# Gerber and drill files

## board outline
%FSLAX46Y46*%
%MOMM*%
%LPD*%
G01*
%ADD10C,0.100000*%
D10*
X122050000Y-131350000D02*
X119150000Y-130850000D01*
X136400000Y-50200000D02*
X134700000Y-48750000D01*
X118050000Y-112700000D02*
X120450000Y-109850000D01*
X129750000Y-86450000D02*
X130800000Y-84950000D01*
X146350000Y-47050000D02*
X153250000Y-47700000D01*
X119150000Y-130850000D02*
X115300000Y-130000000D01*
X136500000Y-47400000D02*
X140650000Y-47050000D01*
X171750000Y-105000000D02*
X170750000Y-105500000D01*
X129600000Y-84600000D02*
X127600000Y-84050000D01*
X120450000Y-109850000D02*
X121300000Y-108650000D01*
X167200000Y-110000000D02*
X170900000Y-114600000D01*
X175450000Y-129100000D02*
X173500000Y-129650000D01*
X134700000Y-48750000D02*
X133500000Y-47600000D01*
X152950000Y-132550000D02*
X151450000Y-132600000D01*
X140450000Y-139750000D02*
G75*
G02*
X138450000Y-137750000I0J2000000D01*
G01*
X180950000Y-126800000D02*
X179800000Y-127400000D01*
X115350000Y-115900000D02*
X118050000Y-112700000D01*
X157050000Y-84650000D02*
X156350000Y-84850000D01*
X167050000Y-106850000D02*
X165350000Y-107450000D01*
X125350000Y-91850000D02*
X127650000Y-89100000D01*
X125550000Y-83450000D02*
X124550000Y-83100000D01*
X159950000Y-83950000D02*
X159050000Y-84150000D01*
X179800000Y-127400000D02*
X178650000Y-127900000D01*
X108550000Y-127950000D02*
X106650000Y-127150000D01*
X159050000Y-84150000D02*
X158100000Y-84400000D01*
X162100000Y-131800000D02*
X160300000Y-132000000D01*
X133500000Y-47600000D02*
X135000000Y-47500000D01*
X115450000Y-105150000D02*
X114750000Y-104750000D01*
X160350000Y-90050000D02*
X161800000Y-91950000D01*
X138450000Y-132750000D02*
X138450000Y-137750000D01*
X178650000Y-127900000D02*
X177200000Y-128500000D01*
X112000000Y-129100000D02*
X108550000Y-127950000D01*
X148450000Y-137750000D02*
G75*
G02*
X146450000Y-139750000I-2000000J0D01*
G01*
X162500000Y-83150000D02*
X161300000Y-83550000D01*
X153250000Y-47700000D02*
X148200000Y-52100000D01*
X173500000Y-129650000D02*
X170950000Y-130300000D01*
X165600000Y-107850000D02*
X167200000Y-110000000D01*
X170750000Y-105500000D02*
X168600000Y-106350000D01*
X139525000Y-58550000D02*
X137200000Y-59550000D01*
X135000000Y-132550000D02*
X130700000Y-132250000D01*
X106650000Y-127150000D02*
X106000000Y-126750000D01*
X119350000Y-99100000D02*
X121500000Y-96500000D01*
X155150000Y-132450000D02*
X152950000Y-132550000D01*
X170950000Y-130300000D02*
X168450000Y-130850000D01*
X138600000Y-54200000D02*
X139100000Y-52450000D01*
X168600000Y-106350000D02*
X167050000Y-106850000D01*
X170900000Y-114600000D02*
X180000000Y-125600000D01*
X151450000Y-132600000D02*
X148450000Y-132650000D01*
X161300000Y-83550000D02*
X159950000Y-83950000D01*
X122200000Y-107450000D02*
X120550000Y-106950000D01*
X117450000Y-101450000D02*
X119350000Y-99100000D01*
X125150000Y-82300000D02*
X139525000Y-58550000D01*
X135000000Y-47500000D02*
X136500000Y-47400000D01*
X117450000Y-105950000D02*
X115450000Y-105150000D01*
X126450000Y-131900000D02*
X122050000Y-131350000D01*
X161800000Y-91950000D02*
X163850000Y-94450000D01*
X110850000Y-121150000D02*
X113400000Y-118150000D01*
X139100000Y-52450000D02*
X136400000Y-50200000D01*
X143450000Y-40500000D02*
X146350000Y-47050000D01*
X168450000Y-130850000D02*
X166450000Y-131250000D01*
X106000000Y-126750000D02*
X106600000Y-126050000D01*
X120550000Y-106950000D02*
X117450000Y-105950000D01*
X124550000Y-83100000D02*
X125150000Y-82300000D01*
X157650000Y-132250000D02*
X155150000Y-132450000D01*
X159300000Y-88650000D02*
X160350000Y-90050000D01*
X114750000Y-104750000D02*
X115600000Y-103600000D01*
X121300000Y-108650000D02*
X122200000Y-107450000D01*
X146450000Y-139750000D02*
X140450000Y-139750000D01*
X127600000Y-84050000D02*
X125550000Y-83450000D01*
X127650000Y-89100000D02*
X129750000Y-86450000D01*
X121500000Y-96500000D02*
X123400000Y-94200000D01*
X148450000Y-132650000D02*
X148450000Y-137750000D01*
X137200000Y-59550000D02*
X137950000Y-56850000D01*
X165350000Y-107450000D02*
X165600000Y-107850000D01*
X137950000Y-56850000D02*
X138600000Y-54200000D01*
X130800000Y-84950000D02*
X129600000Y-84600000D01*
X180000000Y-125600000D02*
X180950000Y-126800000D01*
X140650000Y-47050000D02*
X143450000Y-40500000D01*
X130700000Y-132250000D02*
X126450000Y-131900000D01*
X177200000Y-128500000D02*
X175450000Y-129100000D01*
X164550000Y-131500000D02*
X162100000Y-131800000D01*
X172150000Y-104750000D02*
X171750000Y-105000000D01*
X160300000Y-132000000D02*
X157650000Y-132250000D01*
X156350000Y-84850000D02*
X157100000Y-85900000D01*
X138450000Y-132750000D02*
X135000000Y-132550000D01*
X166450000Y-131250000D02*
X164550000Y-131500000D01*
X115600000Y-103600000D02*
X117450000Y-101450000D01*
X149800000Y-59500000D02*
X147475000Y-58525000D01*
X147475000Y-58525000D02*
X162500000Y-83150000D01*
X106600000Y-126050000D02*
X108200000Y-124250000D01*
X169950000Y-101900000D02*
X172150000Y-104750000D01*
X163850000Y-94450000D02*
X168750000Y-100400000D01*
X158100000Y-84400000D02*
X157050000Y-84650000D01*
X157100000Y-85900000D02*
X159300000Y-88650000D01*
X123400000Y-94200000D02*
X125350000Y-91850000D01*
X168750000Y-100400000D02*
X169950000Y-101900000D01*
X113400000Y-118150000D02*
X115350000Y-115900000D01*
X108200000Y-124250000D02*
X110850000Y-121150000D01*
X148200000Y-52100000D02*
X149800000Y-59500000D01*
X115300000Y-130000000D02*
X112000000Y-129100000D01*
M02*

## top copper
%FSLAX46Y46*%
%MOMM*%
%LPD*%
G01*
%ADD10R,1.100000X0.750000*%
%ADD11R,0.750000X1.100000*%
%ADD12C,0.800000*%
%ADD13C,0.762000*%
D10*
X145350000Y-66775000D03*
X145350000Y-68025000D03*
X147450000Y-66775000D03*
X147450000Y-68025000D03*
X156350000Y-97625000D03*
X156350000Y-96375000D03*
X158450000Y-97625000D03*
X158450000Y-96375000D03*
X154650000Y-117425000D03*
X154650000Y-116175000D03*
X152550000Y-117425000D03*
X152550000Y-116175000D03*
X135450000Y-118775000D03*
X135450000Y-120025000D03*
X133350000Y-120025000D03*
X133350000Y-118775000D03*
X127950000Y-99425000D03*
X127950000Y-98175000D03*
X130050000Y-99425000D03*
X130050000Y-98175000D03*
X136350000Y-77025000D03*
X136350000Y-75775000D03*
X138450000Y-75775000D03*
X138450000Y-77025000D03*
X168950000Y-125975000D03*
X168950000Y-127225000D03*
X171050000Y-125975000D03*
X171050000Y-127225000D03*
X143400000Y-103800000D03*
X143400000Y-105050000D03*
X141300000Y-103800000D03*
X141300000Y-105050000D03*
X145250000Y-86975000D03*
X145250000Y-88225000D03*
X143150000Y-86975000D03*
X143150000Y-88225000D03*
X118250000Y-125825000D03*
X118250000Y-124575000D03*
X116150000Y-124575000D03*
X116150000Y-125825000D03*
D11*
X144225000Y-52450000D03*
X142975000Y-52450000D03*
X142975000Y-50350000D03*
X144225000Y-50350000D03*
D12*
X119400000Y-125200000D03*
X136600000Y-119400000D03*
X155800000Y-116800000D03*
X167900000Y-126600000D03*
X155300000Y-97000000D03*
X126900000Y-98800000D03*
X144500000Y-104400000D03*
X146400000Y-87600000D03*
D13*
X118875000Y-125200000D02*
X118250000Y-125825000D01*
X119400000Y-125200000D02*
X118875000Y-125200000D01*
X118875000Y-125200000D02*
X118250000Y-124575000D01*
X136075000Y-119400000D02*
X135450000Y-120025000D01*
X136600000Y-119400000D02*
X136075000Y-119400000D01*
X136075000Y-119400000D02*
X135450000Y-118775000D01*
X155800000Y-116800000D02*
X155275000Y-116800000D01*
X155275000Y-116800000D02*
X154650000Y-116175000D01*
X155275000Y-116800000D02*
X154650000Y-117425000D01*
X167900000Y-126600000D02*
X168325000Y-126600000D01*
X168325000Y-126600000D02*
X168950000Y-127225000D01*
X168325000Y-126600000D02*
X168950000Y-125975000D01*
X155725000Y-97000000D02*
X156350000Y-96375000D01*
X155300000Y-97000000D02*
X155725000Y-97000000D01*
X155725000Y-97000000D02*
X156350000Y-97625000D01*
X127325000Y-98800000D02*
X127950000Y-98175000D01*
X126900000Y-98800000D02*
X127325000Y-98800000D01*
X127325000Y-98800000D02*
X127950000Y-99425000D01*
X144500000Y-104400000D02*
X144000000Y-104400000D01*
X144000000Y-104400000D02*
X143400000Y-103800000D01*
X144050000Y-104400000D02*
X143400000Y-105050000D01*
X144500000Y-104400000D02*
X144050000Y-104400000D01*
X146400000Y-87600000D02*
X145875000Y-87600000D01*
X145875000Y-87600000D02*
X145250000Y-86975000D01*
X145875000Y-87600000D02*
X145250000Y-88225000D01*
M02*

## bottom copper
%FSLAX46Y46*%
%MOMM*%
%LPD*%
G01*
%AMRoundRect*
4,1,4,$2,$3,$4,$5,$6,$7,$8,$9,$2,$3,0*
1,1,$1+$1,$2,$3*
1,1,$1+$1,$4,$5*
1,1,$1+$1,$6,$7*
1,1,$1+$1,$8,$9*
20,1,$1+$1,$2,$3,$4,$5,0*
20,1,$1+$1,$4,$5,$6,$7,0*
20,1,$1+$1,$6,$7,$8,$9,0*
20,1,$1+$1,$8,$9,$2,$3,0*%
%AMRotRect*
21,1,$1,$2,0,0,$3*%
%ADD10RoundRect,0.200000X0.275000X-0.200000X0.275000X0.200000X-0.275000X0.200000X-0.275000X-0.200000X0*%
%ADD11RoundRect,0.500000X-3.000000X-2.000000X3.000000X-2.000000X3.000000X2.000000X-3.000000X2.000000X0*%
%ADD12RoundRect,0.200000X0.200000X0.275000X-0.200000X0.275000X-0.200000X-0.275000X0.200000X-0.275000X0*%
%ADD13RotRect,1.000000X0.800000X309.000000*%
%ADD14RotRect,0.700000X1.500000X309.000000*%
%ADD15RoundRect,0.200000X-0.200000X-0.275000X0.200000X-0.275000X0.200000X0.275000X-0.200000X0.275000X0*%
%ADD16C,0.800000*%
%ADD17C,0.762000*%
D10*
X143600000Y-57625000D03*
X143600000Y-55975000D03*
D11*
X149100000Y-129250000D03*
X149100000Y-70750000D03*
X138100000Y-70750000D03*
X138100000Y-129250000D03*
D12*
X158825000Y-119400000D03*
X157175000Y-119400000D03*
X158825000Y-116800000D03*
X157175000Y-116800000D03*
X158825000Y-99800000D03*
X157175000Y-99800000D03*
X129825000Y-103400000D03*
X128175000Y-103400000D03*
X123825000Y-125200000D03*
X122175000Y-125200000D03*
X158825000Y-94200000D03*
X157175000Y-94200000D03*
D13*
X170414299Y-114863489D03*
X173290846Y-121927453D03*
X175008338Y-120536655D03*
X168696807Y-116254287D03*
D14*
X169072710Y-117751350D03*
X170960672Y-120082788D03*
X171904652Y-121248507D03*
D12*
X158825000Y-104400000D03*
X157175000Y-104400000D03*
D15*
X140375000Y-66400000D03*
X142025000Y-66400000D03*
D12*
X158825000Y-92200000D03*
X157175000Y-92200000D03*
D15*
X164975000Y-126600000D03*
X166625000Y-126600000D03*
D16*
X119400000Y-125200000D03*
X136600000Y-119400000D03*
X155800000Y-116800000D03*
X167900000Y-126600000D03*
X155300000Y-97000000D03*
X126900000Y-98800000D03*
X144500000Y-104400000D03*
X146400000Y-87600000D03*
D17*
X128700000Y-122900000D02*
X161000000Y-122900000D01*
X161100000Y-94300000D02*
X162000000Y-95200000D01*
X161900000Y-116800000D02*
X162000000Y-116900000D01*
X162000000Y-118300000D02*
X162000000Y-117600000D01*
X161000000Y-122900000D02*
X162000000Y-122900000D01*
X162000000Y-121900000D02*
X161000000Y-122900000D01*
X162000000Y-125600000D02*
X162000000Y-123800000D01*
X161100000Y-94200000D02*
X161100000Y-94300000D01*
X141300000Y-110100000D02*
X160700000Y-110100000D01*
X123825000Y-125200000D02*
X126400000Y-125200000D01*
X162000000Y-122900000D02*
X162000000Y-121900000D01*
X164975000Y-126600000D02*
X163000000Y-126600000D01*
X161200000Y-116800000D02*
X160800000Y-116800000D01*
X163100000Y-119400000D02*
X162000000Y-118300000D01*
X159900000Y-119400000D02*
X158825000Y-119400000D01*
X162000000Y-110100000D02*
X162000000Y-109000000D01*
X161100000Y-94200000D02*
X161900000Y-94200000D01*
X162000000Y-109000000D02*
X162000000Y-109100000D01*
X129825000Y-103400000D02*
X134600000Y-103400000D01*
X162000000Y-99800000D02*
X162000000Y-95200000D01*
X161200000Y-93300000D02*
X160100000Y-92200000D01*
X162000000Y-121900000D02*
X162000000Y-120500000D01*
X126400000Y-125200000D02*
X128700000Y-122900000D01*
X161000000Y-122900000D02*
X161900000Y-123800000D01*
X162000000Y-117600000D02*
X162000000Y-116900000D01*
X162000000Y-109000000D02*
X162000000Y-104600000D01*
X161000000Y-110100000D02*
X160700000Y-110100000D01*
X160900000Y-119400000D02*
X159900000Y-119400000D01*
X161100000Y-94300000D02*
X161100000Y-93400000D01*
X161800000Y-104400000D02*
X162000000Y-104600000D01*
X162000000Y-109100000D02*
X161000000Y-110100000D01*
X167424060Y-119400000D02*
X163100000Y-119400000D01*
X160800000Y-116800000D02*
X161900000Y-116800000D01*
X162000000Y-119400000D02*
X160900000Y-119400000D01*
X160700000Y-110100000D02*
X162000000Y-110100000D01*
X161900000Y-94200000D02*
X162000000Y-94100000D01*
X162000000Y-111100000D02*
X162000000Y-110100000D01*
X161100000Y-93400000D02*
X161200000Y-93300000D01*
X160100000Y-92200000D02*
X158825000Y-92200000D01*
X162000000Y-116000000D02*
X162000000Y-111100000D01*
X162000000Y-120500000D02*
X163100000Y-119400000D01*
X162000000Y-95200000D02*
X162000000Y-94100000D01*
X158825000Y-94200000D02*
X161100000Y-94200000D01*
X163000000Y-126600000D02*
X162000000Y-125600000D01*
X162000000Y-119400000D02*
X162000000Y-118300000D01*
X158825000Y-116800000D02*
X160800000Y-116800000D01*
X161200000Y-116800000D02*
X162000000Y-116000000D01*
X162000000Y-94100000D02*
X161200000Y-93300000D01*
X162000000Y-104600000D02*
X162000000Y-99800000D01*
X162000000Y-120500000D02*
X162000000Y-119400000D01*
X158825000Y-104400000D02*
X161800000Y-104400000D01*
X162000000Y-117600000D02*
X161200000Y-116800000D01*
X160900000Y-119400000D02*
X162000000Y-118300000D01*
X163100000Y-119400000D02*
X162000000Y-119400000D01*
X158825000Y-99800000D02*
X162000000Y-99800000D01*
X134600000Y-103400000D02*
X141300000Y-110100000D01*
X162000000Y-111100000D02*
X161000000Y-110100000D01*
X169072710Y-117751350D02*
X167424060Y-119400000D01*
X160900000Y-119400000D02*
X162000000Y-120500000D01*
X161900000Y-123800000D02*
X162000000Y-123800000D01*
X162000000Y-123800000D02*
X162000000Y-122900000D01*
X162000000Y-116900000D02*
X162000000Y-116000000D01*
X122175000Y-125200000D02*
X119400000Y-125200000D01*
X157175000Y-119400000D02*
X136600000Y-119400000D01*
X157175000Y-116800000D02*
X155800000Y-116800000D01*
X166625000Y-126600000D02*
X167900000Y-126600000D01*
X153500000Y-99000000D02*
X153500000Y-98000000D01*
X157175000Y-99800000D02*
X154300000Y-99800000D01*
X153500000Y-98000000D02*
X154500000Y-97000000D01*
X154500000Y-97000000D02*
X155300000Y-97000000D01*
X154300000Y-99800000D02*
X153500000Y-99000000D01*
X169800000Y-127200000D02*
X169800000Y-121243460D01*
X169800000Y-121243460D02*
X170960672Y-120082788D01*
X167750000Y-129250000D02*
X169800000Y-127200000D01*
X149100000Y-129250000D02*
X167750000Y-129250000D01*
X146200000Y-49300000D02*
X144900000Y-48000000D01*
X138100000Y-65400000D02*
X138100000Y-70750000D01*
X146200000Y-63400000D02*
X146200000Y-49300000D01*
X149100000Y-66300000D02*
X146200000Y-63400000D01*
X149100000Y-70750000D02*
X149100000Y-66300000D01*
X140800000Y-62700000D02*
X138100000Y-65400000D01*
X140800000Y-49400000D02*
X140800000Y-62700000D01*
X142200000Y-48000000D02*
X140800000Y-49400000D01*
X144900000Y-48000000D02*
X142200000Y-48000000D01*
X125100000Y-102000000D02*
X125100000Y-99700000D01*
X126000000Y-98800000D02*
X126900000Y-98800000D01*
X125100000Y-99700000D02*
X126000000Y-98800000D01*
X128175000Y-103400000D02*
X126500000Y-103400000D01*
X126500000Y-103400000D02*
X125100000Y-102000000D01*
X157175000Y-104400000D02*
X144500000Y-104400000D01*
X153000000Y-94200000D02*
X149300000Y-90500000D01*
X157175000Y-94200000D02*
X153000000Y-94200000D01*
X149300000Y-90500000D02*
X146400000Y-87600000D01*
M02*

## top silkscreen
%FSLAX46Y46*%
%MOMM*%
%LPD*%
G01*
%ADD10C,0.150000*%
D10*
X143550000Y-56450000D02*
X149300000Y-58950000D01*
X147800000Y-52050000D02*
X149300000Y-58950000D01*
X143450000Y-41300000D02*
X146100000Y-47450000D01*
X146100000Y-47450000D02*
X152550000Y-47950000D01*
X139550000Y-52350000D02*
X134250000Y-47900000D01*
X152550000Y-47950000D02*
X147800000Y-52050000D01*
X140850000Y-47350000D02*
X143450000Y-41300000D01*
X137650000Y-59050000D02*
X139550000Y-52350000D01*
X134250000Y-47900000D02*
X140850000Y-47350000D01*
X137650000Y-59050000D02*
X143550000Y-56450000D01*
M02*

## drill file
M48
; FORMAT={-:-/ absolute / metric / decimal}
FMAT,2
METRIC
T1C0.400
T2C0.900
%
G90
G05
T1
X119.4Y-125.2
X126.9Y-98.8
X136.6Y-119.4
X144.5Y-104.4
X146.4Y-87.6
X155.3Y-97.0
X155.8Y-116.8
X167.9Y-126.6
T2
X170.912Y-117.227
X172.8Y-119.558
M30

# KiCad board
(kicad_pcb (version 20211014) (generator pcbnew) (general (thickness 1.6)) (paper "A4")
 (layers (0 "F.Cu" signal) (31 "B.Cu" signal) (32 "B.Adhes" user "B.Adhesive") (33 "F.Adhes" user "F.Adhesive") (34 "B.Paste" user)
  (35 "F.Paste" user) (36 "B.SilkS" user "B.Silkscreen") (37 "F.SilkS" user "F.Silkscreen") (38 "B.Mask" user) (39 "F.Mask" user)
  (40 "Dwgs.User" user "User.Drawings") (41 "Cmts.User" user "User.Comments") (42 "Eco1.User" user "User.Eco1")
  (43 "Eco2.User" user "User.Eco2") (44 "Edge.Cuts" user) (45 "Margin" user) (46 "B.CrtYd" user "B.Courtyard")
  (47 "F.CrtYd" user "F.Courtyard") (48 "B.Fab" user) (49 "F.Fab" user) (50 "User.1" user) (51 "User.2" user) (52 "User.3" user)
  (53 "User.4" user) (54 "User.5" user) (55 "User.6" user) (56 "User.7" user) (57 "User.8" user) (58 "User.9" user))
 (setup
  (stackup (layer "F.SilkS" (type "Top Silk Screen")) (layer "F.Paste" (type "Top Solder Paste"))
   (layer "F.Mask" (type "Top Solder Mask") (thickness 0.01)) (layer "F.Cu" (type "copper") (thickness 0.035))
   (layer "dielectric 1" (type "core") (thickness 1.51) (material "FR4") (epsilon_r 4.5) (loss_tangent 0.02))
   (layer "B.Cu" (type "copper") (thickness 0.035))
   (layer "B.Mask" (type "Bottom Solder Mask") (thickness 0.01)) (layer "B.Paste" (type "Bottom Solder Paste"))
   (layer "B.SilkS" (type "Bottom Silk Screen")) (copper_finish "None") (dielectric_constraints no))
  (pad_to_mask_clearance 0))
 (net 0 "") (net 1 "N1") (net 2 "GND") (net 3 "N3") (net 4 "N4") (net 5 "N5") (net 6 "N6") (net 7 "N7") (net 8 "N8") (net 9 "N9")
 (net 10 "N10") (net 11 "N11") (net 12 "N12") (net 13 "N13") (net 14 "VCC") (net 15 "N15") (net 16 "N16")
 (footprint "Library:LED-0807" (layer "F.Cu") (at 146.4 67.4)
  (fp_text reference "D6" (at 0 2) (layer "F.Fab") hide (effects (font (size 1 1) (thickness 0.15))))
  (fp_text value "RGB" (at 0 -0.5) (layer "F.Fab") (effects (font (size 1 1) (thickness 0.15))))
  (pad "1" smd rect locked (at -1.05 -0.625) (size 1.1 0.75) (layers "F.Cu" "F.Paste" "F.Mask") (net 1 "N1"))
  (pad "1" smd rect locked (at -1.05 0.625) (size 1.1 0.75) (layers "F.Cu" "F.Paste" "F.Mask") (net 1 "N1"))
  (pad "2" smd rect locked (at 1.05 -0.625) (size 1.1 0.75) (layers "F.Cu" "F.Paste" "F.Mask") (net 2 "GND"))
  (pad "2" smd rect locked (at 1.05 0.625) (size 1.1 0.75) (layers "F.Cu" "F.Paste" "F.Mask") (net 2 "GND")))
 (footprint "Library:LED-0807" (layer "F.Cu") (at 157.4 97)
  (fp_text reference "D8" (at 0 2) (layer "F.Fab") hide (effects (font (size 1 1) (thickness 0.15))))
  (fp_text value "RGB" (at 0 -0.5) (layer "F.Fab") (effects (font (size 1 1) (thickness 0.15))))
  (pad "1" smd rect locked (at -1.05 0.625) (size 1.1 0.75) (layers "F.Cu" "F.Paste" "F.Mask") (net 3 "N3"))
  (pad "1" smd rect locked (at -1.05 -0.625) (size 1.1 0.75) (layers "F.Cu" "F.Paste" "F.Mask") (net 3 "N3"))
  (pad "2" smd rect locked (at 1.05 0.625) (size 1.1 0.75) (layers "F.Cu" "F.Paste" "F.Mask") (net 2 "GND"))
  (pad "2" smd rect locked (at 1.05 -0.625) (size 1.1 0.75) (layers "F.Cu" "F.Paste" "F.Mask") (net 2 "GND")))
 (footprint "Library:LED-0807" (layer "F.Cu") (at 153.6 116.8 180)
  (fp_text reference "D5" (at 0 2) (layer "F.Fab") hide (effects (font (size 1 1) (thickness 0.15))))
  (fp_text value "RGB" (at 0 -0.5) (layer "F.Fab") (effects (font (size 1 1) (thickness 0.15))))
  (pad "1" smd rect locked (at -1.05 -0.625 180) (size 1.1 0.75) (layers "F.Cu" "F.Paste" "F.Mask") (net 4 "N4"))
  (pad "1" smd rect locked (at -1.05 0.625 180) (size 1.1 0.75) (layers "F.Cu" "F.Paste" "F.Mask") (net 4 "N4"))
  (pad "2" smd rect locked (at 1.05 -0.625 180) (size 1.1 0.75) (layers "F.Cu" "F.Paste" "F.Mask") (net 2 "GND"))
  (pad "2" smd rect locked (at 1.05 0.625 180) (size 1.1 0.75) (layers "F.Cu" "F.Paste" "F.Mask") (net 2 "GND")))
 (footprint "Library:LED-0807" (layer "F.Cu") (at 134.4 119.4 180)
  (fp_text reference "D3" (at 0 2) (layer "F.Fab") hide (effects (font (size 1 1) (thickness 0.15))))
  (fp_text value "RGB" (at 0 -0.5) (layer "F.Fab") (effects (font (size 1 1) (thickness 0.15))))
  (pad "1" smd rect locked (at -1.05 0.625 180) (size 1.1 0.75) (layers "F.Cu" "F.Paste" "F.Mask") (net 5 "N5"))
  (pad "1" smd rect locked (at -1.05 -0.625 180) (size 1.1 0.75) (layers "F.Cu" "F.Paste" "F.Mask") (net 5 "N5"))
  (pad "2" smd rect locked (at 1.05 -0.625 180) (size 1.1 0.75) (layers "F.Cu" "F.Paste" "F.Mask") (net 2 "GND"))
  (pad "2" smd rect locked (at 1.05 0.625 180) (size 1.1 0.75) (layers "F.Cu" "F.Paste" "F.Mask") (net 2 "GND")))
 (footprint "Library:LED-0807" (layer "F.Cu") (at 129 98.8)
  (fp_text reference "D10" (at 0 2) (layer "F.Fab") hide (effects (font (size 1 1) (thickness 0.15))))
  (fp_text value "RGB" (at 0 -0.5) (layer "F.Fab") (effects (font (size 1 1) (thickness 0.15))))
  (pad "1" smd rect locked (at -1.05 0.625) (size 1.1 0.75) (layers "F.Cu" "F.Paste" "F.Mask") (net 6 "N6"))
  (pad "1" smd rect locked (at -1.05 -0.625) (size 1.1 0.75) (layers "F.Cu" "F.Paste" "F.Mask") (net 6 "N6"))
  (pad "2" smd rect locked (at 1.05 0.625) (size 1.1 0.75) (layers "F.Cu" "F.Paste" "F.Mask") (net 2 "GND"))
  (pad "2" smd rect locked (at 1.05 -0.625) (size 1.1 0.75) (layers "F.Cu" "F.Paste" "F.Mask") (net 2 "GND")))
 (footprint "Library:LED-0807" (layer "F.Cu") (at 137.4 76.4)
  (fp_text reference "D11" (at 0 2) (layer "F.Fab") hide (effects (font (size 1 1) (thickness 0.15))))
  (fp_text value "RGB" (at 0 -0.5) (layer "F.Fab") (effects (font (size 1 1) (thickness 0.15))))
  (pad "1" smd rect locked (at -1.05 0.625) (size 1.1 0.75) (layers "F.Cu" "F.Paste" "F.Mask") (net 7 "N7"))
  (pad "1" smd rect locked (at -1.05 -0.625) (size 1.1 0.75) (layers "F.Cu" "F.Paste" "F.Mask") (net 7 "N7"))
  (pad "2" smd rect locked (at 1.05 -0.625) (size 1.1 0.75) (layers "F.Cu" "F.Paste" "F.Mask") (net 2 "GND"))
  (pad "2" smd rect locked (at 1.05 0.625) (size 1.1 0.75) (layers "F.Cu" "F.Paste" "F.Mask") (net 2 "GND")))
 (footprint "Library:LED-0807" (layer "F.Cu") (at 170 126.6)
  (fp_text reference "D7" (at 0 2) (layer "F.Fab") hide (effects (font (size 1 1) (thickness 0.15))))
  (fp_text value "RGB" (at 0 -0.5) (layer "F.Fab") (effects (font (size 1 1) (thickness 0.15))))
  (pad "1" smd rect locked (at -1.05 -0.625) (size 1.1 0.75) (layers "F.Cu" "F.Paste" "F.Mask") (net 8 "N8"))
  (pad "1" smd rect locked (at -1.05 0.625) (size 1.1 0.75) (layers "F.Cu" "F.Paste" "F.Mask") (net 8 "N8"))
  (pad "2" smd rect locked (at 1.05 -0.625) (size 1.1 0.75) (layers "F.Cu" "F.Paste" "F.Mask") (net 2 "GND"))
  (pad "2" smd rect locked (at 1.05 0.625) (size 1.1 0.75) (layers "F.Cu" "F.Paste" "F.Mask") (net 2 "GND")))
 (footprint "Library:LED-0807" (layer "F.Cu") (at 142.35 104.425 180)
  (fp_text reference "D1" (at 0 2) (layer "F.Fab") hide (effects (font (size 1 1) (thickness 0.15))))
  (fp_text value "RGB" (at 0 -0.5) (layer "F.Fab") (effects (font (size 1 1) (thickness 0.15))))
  (pad "1" smd rect locked (at -1.05 0.625 180) (size 1.1 0.75) (layers "F.Cu" "F.Paste" "F.Mask") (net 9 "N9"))
  (pad "1" smd rect locked (at -1.05 -0.625 180) (size 1.1 0.75) (layers "F.Cu" "F.Paste" "F.Mask") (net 9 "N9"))
  (pad "2" smd rect locked (at 1.05 0.625 180) (size 1.1 0.75) (layers "F.Cu" "F.Paste" "F.Mask") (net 2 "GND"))
  (pad "2" smd rect locked (at 1.05 -0.625 180) (size 1.1 0.75) (layers "F.Cu" "F.Paste" "F.Mask") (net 2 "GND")))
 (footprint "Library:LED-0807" (layer "F.Cu") (at 144.2 87.6 180)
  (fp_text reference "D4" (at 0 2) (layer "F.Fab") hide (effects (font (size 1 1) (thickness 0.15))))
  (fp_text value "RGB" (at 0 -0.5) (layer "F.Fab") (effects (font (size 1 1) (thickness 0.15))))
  (pad "1" smd rect locked (at -1.05 0.625 180) (size 1.1 0.75) (layers "F.Cu" "F.Paste" "F.Mask") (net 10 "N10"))
  (pad "1" smd rect locked (at -1.05 -0.625 180) (size 1.1 0.75) (layers "F.Cu" "F.Paste" "F.Mask") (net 10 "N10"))
  (pad "2" smd rect locked (at 1.05 0.625 180) (size 1.1 0.75) (layers "F.Cu" "F.Paste" "F.Mask") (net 2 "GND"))
  (pad "2" smd rect locked (at 1.05 -0.625 180) (size 1.1 0.75) (layers "F.Cu" "F.Paste" "F.Mask") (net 2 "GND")))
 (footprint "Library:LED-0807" (layer "F.Cu") (at 117.2 125.2 180)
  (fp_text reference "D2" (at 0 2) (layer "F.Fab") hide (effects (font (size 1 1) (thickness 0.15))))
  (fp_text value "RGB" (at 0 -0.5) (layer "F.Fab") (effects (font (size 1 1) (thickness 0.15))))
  (pad "1" smd rect locked (at -1.05 -0.625 180) (size 1.1 0.75) (layers "F.Cu" "F.Paste" "F.Mask") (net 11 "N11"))
  (pad "1" smd rect locked (at -1.05 0.625 180) (size 1.1 0.75) (layers "F.Cu" "F.Paste" "F.Mask") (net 11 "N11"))
  (pad "2" smd rect locked (at 1.05 0.625 180) (size 1.1 0.75) (layers "F.Cu" "F.Paste" "F.Mask") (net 2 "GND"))
  (pad "2" smd rect locked (at 1.05 -0.625 180) (size 1.1 0.75) (layers "F.Cu" "F.Paste" "F.Mask") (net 2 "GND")))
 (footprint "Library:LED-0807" (layer "F.Cu") (at 143.6 51.4 90)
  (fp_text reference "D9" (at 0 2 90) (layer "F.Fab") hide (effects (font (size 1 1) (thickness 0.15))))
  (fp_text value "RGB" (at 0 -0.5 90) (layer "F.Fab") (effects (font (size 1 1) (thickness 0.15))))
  (pad "1" smd rect locked (at -1.05 0.625 90) (size 1.1 0.75) (layers "F.Cu" "F.Paste" "F.Mask") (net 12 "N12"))
  (pad "1" smd rect locked (at -1.05 -0.625 90) (size 1.1 0.75) (layers "F.Cu" "F.Paste" "F.Mask") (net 12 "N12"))
  (pad "2" smd rect locked (at 1.05 -0.625 90) (size 1.1 0.75) (layers "F.Cu" "F.Paste" "F.Mask") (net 2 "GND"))
  (pad "2" smd rect locked (at 1.05 0.625 90) (size 1.1 0.75) (layers "F.Cu" "F.Paste" "F.Mask") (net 2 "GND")))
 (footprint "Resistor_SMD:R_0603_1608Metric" (layer "B.Cu") (at 143.6 56.8 90)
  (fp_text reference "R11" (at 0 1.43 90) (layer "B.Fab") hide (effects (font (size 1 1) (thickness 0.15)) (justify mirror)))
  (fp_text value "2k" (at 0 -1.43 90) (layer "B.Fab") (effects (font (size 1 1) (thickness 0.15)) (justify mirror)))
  (pad "1" smd roundrect locked (at -0.825 0 90) (size 0.8 0.95) (layers "B.Cu" "B.Paste" "B.Mask") (roundrect_rratio 0.25) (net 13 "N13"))
  (pad "2" smd roundrect locked (at 0.825 0 90) (size 0.8 0.95) (layers "B.Cu" "B.Paste" "B.Mask") (roundrect_rratio 0.25) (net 12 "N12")))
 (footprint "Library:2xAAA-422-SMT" (layer "B.Cu") (at 143.6 100)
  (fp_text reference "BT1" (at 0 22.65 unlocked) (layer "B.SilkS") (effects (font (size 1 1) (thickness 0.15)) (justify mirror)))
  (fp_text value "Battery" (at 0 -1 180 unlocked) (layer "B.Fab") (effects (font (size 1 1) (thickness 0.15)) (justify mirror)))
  (pad "1" smd roundrect (at 5.5 29.25) (size 7 5) (layers "B.Cu" "B.Paste" "B.Mask") (roundrect_rratio 0.1) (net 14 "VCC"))
  (pad "2" smd roundrect (at 5.5 -29.25) (size 7 5) (layers "B.Cu" "B.Paste" "B.Mask") (roundrect_rratio 0.1) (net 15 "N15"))
  (pad "2" smd roundrect (at -5.5 -29.25) (size 7 5) (layers "B.Cu" "B.Paste" "B.Mask") (roundrect_rratio 0.1) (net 15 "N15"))
  (pad "3" smd roundrect (at -5.5 29.25) (size 7 5) (layers "B.Cu" "B.Paste" "B.Mask") (roundrect_rratio 0.1) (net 2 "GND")))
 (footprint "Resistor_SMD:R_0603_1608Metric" (layer "B.Cu") (at 158 119.4 180)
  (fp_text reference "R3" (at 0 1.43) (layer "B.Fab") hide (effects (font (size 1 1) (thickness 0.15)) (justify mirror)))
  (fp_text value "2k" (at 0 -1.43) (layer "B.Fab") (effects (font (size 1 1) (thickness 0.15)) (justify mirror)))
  (pad "1" smd roundrect locked (at -0.825 0 180) (size 0.8 0.95) (layers "B.Cu" "B.Paste" "B.Mask") (roundrect_rratio 0.25) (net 13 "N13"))
  (pad "2" smd roundrect locked (at 0.825 0 180) (size 0.8 0.95) (layers "B.Cu" "B.Paste" "B.Mask") (roundrect_rratio 0.25) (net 5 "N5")))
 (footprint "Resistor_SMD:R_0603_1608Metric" (layer "B.Cu") (at 158 116.8 180)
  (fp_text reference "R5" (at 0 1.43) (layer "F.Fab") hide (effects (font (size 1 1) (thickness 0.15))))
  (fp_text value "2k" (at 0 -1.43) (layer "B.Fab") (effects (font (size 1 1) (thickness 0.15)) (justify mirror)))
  (pad "1" smd roundrect locked (at -0.825 0 180) (size 0.8 0.95) (layers "B.Cu" "B.Paste" "B.Mask") (roundrect_rratio 0.25) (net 13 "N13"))
  (pad "2" smd roundrect locked (at 0.825 0 180) (size 0.8 0.95) (layers "B.Cu" "B.Paste" "B.Mask") (roundrect_rratio 0.25) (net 4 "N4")))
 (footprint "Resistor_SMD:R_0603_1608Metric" (layer "B.Cu") (at 158 99.8 180)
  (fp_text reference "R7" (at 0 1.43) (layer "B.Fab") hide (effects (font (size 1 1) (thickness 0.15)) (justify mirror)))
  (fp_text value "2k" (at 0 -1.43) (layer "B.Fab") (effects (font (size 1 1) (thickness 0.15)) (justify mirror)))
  (pad "1" smd roundrect locked (at -0.825 0 180) (size 0.8 0.95) (layers "B.Cu" "B.Paste" "B.Mask") (roundrect_rratio 0.25) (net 13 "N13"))
  (pad "2" smd roundrect locked (at 0.825 0 180) (size 0.8 0.95) (layers "B.Cu" "B.Paste" "B.Mask") (roundrect_rratio 0.25) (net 3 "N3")))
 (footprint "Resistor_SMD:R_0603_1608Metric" (layer "B.Cu") (at 129 103.4 180)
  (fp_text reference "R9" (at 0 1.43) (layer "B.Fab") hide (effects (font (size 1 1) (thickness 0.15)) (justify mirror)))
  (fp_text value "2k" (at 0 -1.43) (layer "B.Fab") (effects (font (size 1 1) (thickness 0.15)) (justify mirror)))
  (pad "1" smd roundrect locked (at -0.825 0 180) (size 0.8 0.95) (layers "B.Cu" "B.Paste" "B.Mask") (roundrect_rratio 0.25) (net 13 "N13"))
  (pad "2" smd roundrect locked (at 0.825 0 180) (size 0.8 0.95) (layers "B.Cu" "B.Paste" "B.Mask") (roundrect_rratio 0.25) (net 6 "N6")))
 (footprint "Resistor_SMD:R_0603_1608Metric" (layer "B.Cu") (at 123 125.2 180)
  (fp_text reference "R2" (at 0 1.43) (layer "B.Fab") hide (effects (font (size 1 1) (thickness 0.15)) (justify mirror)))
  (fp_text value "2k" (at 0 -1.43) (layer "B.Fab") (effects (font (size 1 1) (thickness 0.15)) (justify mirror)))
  (pad "1" smd roundrect locked (at -0.825 0 180) (size 0.8 0.95) (layers "B.Cu" "B.Paste" "B.Mask") (roundrect_rratio 0.25) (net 13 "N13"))
  (pad "2" smd roundrect locked (at 0.825 0 180) (size 0.8 0.95) (layers "B.Cu" "B.Paste" "B.Mask") (roundrect_rratio 0.25) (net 11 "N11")))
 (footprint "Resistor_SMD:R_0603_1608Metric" (layer "B.Cu") (at 158 94.2 180)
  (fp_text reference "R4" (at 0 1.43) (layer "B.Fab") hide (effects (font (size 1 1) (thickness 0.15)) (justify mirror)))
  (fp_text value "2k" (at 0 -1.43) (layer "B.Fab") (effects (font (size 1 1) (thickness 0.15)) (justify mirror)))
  (pad "1" smd roundrect locked (at -0.825 0 180) (size 0.8 0.95) (layers "B.Cu" "B.Paste" "B.Mask") (roundrect_rratio 0.25) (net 13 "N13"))
  (pad "2" smd roundrect locked (at 0.825 0 180) (size 0.8 0.95) (layers "B.Cu" "B.Paste" "B.Mask") (roundrect_rratio 0.25) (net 10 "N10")))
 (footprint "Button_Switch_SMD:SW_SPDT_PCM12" (layer "B.Cu") (at 171.6 118.6 -51)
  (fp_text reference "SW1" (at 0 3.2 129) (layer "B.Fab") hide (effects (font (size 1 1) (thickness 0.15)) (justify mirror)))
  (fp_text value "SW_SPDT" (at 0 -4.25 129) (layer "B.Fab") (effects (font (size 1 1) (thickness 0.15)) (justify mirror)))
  (pad "" smd rect locked (at -3.65 -1.43 309) (size 1 0.8) (layers "B.Cu" "B.Paste" "B.Mask"))
  (pad "" np_thru_hole circle locked (at 1.5 -0.33 309) (size 0.9 0.9) (drill 0.9) (layers *.Cu *.Mask))
  (pad "" smd rect locked (at 3.65 0.78 309) (size 1 0.8) (layers "B.Cu" "B.Paste" "B.Mask"))
  (pad "" np_thru_hole circle locked (at -1.5 -0.33 309) (size 0.9 0.9) (drill 0.9) (layers *.Cu *.Mask))
  (pad "" smd rect locked (at 3.65 -1.43 309) (size 1 0.8) (layers "B.Cu" "B.Paste" "B.Mask"))
  (pad "" smd rect locked (at -3.65 0.78 309) (size 1 0.8) (layers "B.Cu" "B.Paste" "B.Mask"))
  (pad "1" smd rect locked (at -2.25 1.43 309) (size 0.7 1.5) (layers "B.Cu" "B.Paste" "B.Mask") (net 13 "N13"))
  (pad "2" smd rect locked (at 0.75 1.43 309) (size 0.7 1.5) (layers "B.Cu" "B.Paste" "B.Mask") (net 14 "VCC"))
  (pad "3" smd rect locked (at 2.25 1.43 309) (size 0.7 1.5) (layers "B.Cu" "B.Paste" "B.Mask") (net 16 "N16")))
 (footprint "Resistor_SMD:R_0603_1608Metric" (layer "B.Cu") (at 158 104.4 180)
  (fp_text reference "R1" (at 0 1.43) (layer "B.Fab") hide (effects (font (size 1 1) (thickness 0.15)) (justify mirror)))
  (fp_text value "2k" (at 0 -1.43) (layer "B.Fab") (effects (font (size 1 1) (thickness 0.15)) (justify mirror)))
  (pad "1" smd roundrect locked (at -0.825 0 180) (size 0.8 0.95) (layers "B.Cu" "B.Paste" "B.Mask") (roundrect_rratio 0.25) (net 13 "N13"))
  (pad "2" smd roundrect locked (at 0.825 0 180) (size 0.8 0.95) (layers "B.Cu" "B.Paste" "B.Mask") (roundrect_rratio 0.25) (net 9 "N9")))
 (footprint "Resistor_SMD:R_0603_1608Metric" (layer "B.Cu") (at 141.2 66.4)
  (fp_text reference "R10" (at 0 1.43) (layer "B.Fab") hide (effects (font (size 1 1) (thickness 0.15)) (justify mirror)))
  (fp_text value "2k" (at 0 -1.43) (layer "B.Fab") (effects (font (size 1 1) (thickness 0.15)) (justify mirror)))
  (pad "1" smd roundrect locked (at -0.825 0) (size 0.8 0.95) (layers "B.Cu" "B.Paste" "B.Mask") (roundrect_rratio 0.25) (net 13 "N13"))
  (pad "2" smd roundrect locked (at 0.825 0) (size 0.8 0.95) (layers "B.Cu" "B.Paste" "B.Mask") (roundrect_rratio 0.25) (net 1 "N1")))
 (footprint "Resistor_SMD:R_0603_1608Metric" (layer "B.Cu") (at 158 92.2 180)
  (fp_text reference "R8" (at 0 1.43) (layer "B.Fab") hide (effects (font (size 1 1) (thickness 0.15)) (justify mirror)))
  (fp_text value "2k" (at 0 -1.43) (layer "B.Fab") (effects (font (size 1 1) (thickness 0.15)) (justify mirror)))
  (pad "1" smd roundrect locked (at -0.825 0 180) (size 0.8 0.95) (layers "B.Cu" "B.Paste" "B.Mask") (roundrect_rratio 0.25) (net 13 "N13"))
  (pad "2" smd roundrect locked (at 0.825 0 180) (size 0.8 0.95) (layers "B.Cu" "B.Paste" "B.Mask") (roundrect_rratio 0.25) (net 7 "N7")))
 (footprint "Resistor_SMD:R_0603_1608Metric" (layer "B.Cu") (at 165.8 126.6)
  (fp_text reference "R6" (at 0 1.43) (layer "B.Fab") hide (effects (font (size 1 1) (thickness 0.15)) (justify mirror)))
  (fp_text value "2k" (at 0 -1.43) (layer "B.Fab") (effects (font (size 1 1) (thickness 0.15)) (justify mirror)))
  (pad "1" smd roundrect locked (at -0.825 0) (size 0.8 0.95) (layers "B.Cu" "B.Paste" "B.Mask") (roundrect_rratio 0.25) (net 13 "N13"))
  (pad "2" smd roundrect locked (at 0.825 0) (size 0.8 0.95) (layers "B.Cu" "B.Paste" "B.Mask") (roundrect_rratio 0.25) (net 8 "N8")))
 (gr_line (start 143.55 56.45) (end 149.3 58.95) (layer "F.SilkS") (width 0.15))
 (gr_line (start 147.8 52.05) (end 149.3 58.95) (layer "F.SilkS") (width 0.15))
 (gr_line (start 143.45 41.3) (end 146.1 47.45) (layer "F.SilkS") (width 0.15))
 (gr_line (start 146.1 47.45) (end 152.55 47.95) (layer "F.SilkS") (width 0.15))
 (gr_line (start 139.55 52.35) (end 134.25 47.9) (layer "F.SilkS") (width 0.15))
 (gr_line (start 152.55 47.95) (end 147.8 52.05) (layer "F.SilkS") (width 0.15))
 (gr_line (start 140.85 47.35) (end 143.45 41.3) (layer "F.SilkS") (width 0.15))
 (gr_line (start 137.65 59.05) (end 139.55 52.35) (layer "F.SilkS") (width 0.15))
 (gr_line (start 134.25 47.9) (end 140.85 47.35) (layer "F.SilkS") (width 0.15))
 (gr_line (start 137.65 59.05) (end 143.55 56.45) (layer "F.SilkS") (width 0.15))
 (gr_line (start 122.05 131.35) (end 119.15 130.85) (layer "Edge.Cuts") (width 0.1))
 (gr_line (start 136.4 50.2) (end 134.7 48.75) (layer "Edge.Cuts") (width 0.1))
 (gr_line (start 118.05 112.7) (end 120.45 109.85) (layer "Edge.Cuts") (width 0.1))
 (gr_line (start 129.75 86.45) (end 130.8 84.95) (layer "Edge.Cuts") (width 0.1))
 (gr_line (start 146.35 47.05) (end 153.25 47.7) (layer "Edge.Cuts") (width 0.1))
 (gr_line (start 119.15 130.85) (end 115.3 130) (layer "Edge.Cuts") (width 0.1))
 (gr_line (start 136.5 47.4) (end 140.65 47.05) (layer "Edge.Cuts") (width 0.1))
 (gr_line (start 171.75 105) (end 170.75 105.5) (layer "Edge.Cuts") (width 0.1))
 (gr_line (start 129.6 84.6) (end 127.6 84.05) (layer "Edge.Cuts") (width 0.1))
 (gr_line (start 120.45 109.85) (end 121.3 108.65) (layer "Edge.Cuts") (width 0.1))
 (gr_line (start 167.2 110) (end 170.9 114.6) (layer "Edge.Cuts") (width 0.1))
 (gr_line (start 175.45 129.1) (end 173.5 129.65) (layer "Edge.Cuts") (width 0.1))
 (gr_line (start 134.7 48.75) (end 133.5 47.6) (layer "Edge.Cuts") (width 0.1))
 (gr_line (start 152.95 132.55) (end 151.45 132.6) (layer "Edge.Cuts") (width 0.1))
 (gr_arc (start 140.45 139.75) (mid 139.035786 139.164214) (end 138.45 137.75) (layer "Edge.Cuts") (width 0.1))
 (gr_line (start 180.95 126.8) (end 179.8 127.4) (layer "Edge.Cuts") (width 0.1))
 (gr_line (start 115.35 115.9) (end 118.05 112.7) (layer "Edge.Cuts") (width 0.1))
 (gr_line (start 157.05 84.65) (end 156.35 84.85) (layer "Edge.Cuts") (width 0.1))
 (gr_line (start 167.05 106.85) (end 165.35 107.45) (layer "Edge.Cuts") (width 0.1))
 (gr_line (start 125.35 91.85) (end 127.65 89.1) (layer "Edge.Cuts") (width 0.1))
 (gr_line (start 125.55 83.45) (end 124.55 83.1) (layer "Edge.Cuts") (width 0.1))
 (gr_line (start 159.95 83.95) (end 159.05 84.15) (layer "Edge.Cuts") (width 0.1))
 (gr_line (start 179.8 127.4) (end 178.65 127.9) (layer "Edge.Cuts") (width 0.1))
 (gr_line (start 108.55 127.95) (end 106.65 127.15) (layer "Edge.Cuts") (width 0.1))
 (gr_line (start 159.05 84.15) (end 158.1 84.4) (layer "Edge.Cuts") (width 0.1))
 (gr_line (start 162.1 131.8) (end 160.3 132) (layer "Edge.Cuts") (width 0.1))
 (gr_line (start 133.5 47.6) (end 135 47.5) (layer "Edge.Cuts") (width 0.1))
 (gr_line (start 115.45 105.15) (end 114.75 104.75) (layer "Edge.Cuts") (width 0.1))
 (gr_line (start 160.35 90.05) (end 161.8 91.95) (layer "Edge.Cuts") (width 0.1))
 (gr_line (start 138.45 132.75) (end 138.45 137.75) (layer "Edge.Cuts") (width 0.1))
 (gr_line (start 178.65 127.9) (end 177.2 128.5) (layer "Edge.Cuts") (width 0.1))
 (gr_line (start 112 129.1) (end 108.55 127.95) (layer "Edge.Cuts") (width 0.1))
 (gr_arc (start 148.45 137.75) (mid 147.864214 139.164214) (end 146.45 139.75) (layer "Edge.Cuts") (width 0.1))
 (gr_line (start 162.5 83.15) (end 161.3 83.55) (layer "Edge.Cuts") (width 0.1))
 (gr_line (start 153.25 47.7) (end 148.2 52.1) (layer "Edge.Cuts") (width 0.1))
 (gr_line (start 173.5 129.65) (end 170.95 130.3) (layer "Edge.Cuts") (width 0.1))
 (gr_line (start 165.6 107.85) (end 167.2 110) (layer "Edge.Cuts") (width 0.1))
 (gr_line (start 170.75 105.5) (end 168.6 106.35) (layer "Edge.Cuts") (width 0.1))
 (gr_line (start 139.525 58.55) (end 137.2 59.55) (layer "Edge.Cuts") (width 0.1))
 (gr_line (start 135 132.55) (end 130.7 132.25) (layer "Edge.Cuts") (width 0.1))
 (gr_line (start 106.65 127.15) (end 106 126.75) (layer "Edge.Cuts") (width 0.1))
 (gr_line (start 119.35 99.1) (end 121.5 96.5) (layer "Edge.Cuts") (width 0.1))
 (gr_line (start 155.15 132.45) (end 152.95 132.55) (layer "Edge.Cuts") (width 0.1))
 (gr_line (start 170.95 130.3) (end 168.45 130.85) (layer "Edge.Cuts") (width 0.1))
 (gr_line (start 138.6 54.2) (end 139.1 52.45) (layer "Edge.Cuts") (width 0.1))
 (gr_line (start 168.6 106.35) (end 167.05 106.85) (layer "Edge.Cuts") (width 0.1))
 (gr_line (start 170.9 114.6) (end 180 125.6) (layer "Edge.Cuts") (width 0.1))
 (gr_line (start 151.45 132.6) (end 148.45 132.65) (layer "Edge.Cuts") (width 0.1))
 (gr_line (start 161.3 83.55) (end 159.95 83.95) (layer "Edge.Cuts") (width 0.1))
 (gr_line (start 122.2 107.45) (end 120.55 106.95) (layer "Edge.Cuts") (width 0.1))
 (gr_line (start 117.45 101.45) (end 119.35 99.1) (layer "Edge.Cuts") (width 0.1))
 (gr_line (start 125.15 82.3) (end 139.525 58.55) (layer "Edge.Cuts") (width 0.1))
 (gr_line (start 135 47.5) (end 136.5 47.4) (layer "Edge.Cuts") (width 0.1))
 (gr_line (start 117.45 105.95) (end 115.45 105.15) (layer "Edge.Cuts") (width 0.1))
 (gr_line (start 126.45 131.9) (end 122.05 131.35) (layer "Edge.Cuts") (width 0.1))
 (gr_line (start 161.8 91.95) (end 163.85 94.45) (layer "Edge.Cuts") (width 0.1))
 (gr_line (start 110.85 121.15) (end 113.4 118.15) (layer "Edge.Cuts") (width 0.1))
 (gr_line (start 139.1 52.45) (end 136.4 50.2) (layer "Edge.Cuts") (width 0.1))
 (gr_line (start 143.45 40.5) (end 146.35 47.05) (layer "Edge.Cuts") (width 0.1))
 (gr_line (start 168.45 130.85) (end 166.45 131.25) (layer "Edge.Cuts") (width 0.1))
 (gr_line (start 106 126.75) (end 106.6 126.05) (layer "Edge.Cuts") (width 0.1))
 (gr_line (start 120.55 106.95) (end 117.45 105.95) (layer "Edge.Cuts") (width 0.1))
 (gr_line (start 124.55 83.1) (end 125.15 82.3) (layer "Edge.Cuts") (width 0.1))
 (gr_line (start 157.65 132.25) (end 155.15 132.45) (layer "Edge.Cuts") (width 0.1))
 (gr_line (start 159.3 88.65) (end 160.35 90.05) (layer "Edge.Cuts") (width 0.1))
 (gr_line (start 114.75 104.75) (end 115.6 103.6) (layer "Edge.Cuts") (width 0.1))
 (gr_line (start 121.3 108.65) (end 122.2 107.45) (layer "Edge.Cuts") (width 0.1))
 (gr_line (start 146.45 139.75) (end 140.45 139.75) (layer "Edge.Cuts") (width 0.1))
 (gr_line (start 127.6 84.05) (end 125.55 83.45) (layer "Edge.Cuts") (width 0.1))
 (gr_line (start 127.65 89.1) (end 129.75 86.45) (layer "Edge.Cuts") (width 0.1))
 (gr_line (start 121.5 96.5) (end 123.4 94.2) (layer "Edge.Cuts") (width 0.1))
 (gr_line (start 148.45 132.65) (end 148.45 137.75) (layer "Edge.Cuts") (width 0.1))
 (gr_line (start 137.2 59.55) (end 137.95 56.85) (layer "Edge.Cuts") (width 0.1))
 (gr_line (start 165.35 107.45) (end 165.6 107.85) (layer "Edge.Cuts") (width 0.1))
 (gr_line (start 137.95 56.85) (end 138.6 54.2) (layer "Edge.Cuts") (width 0.1))
 (gr_line (start 130.8 84.95) (end 129.6 84.6) (layer "Edge.Cuts") (width 0.1))
 (gr_line (start 180 125.6) (end 180.95 126.8) (layer "Edge.Cuts") (width 0.1))
 (gr_line (start 140.65 47.05) (end 143.45 40.5) (layer "Edge.Cuts") (width 0.1))
 (gr_line (start 130.7 132.25) (end 126.45 131.9) (layer "Edge.Cuts") (width 0.1))
 (gr_line (start 177.2 128.5) (end 175.45 129.1) (layer "Edge.Cuts") (width 0.1))
 (gr_line (start 164.55 131.5) (end 162.1 131.8) (layer "Edge.Cuts") (width 0.1))
 (gr_line (start 172.15 104.75) (end 171.75 105) (layer "Edge.Cuts") (width 0.1))
 (gr_line (start 160.3 132) (end 157.65 132.25) (layer "Edge.Cuts") (width 0.1))
 (gr_line (start 156.35 84.85) (end 157.1 85.9) (layer "Edge.Cuts") (width 0.1))
 (gr_line (start 138.45 132.75) (end 135 132.55) (layer "Edge.Cuts") (width 0.1))
 (gr_line (start 166.45 131.25) (end 164.55 131.5) (layer "Edge.Cuts") (width 0.1))
 (gr_line (start 115.6 103.6) (end 117.45 101.45) (layer "Edge.Cuts") (width 0.1))
 (gr_line (start 149.8 59.5) (end 147.475 58.525) (layer "Edge.Cuts") (width 0.1))
 (gr_line (start 147.475 58.525) (end 162.5 83.15) (layer "Edge.Cuts") (width 0.1))
 (gr_line (start 106.6 126.05) (end 108.2 124.25) (layer "Edge.Cuts") (width 0.1))
 (gr_line (start 169.95 101.9) (end 172.15 104.75) (layer "Edge.Cuts") (width 0.1))
 (gr_line (start 163.85 94.45) (end 168.75 100.4) (layer "Edge.Cuts") (width 0.1))
 (gr_line (start 158.1 84.4) (end 157.05 84.65) (layer "Edge.Cuts") (width 0.1))
 (gr_line (start 157.1 85.9) (end 159.3 88.65) (layer "Edge.Cuts") (width 0.1))
 (gr_line (start 123.4 94.2) (end 125.35 91.85) (layer "Edge.Cuts") (width 0.1))
 (gr_line (start 168.75 100.4) (end 169.95 101.9) (layer "Edge.Cuts") (width 0.1))
 (gr_line (start 113.4 118.15) (end 115.35 115.9) (layer "Edge.Cuts") (width 0.1))
 (gr_line (start 108.2 124.25) (end 110.85 121.15) (layer "Edge.Cuts") (width 0.1))
 (gr_line (start 148.2 52.1) (end 149.8 59.5) (layer "Edge.Cuts") (width 0.1))
 (gr_line (start 115.3 130) (end 112 129.1) (layer "Edge.Cuts") (width 0.1))
 (segment (start 128.7 122.9) (end 161 122.9) (width 0.762) (layer "B.Cu") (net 13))
 (segment (start 161.1 94.3) (end 162 95.2) (width 0.762) (layer "B.Cu") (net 13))
 (segment (start 161.9 116.8) (end 162 116.9) (width 0.762) (layer "B.Cu") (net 13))
 (segment (start 162 118.3) (end 162 117.6) (width 0.762) (layer "B.Cu") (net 13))
 (segment (start 161 122.9) (end 162 122.9) (width 0.762) (layer "B.Cu") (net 13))
 (segment (start 162 121.9) (end 161 122.9) (width 0.762) (layer "B.Cu") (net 13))
 (segment (start 162 125.6) (end 162 123.8) (width 0.762) (layer "B.Cu") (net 13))
 (segment (start 161.1 94.2) (end 161.1 94.3) (width 0.762) (layer "B.Cu") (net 13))
 (segment (start 141.3 110.1) (end 160.7 110.1) (width 0.762) (layer "B.Cu") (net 13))
 (segment (start 123.825 125.2) (end 126.4 125.2) (width 0.762) (layer "B.Cu") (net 13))
 (segment (start 162 122.9) (end 162 121.9) (width 0.762) (layer "B.Cu") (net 13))
 (segment (start 164.975 126.6) (end 163 126.6) (width 0.762) (layer "B.Cu") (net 13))
 (segment (start 161.2 116.8) (end 160.8 116.8) (width 0.762) (layer "B.Cu") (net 13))
 (segment (start 163.1 119.4) (end 162 118.3) (width 0.762) (layer "B.Cu") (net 13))
 (segment (start 159.9 119.4) (end 158.825 119.4) (width 0.762) (layer "B.Cu") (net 13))
 (segment (start 162 110.1) (end 162 109) (width 0.762) (layer "B.Cu") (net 13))
 (segment (start 161.1 94.2) (end 161.9 94.2) (width 0.762) (layer "B.Cu") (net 13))
 (segment (start 162 109) (end 162 109.1) (width 0.762) (layer "B.Cu") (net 13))
 (segment (start 129.825 103.4) (end 134.6 103.4) (width 0.762) (layer "B.Cu") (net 13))
 (segment (start 162 99.8) (end 162 95.2) (width 0.762) (layer "B.Cu") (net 13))
 (segment (start 161.2 93.3) (end 160.1 92.2) (width 0.762) (layer "B.Cu") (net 13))
 (segment (start 162 121.9) (end 162 120.5) (width 0.762) (layer "B.Cu") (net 13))
 (segment (start 126.4 125.2) (end 128.7 122.9) (width 0.762) (layer "B.Cu") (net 13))
 (segment (start 161 122.9) (end 161.9 123.8) (width 0.762) (layer "B.Cu") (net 13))
 (segment (start 162 117.6) (end 162 116.9) (width 0.762) (layer "B.Cu") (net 13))
 (segment (start 162 109) (end 162 104.6) (width 0.762) (layer "B.Cu") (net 13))
 (segment (start 161 110.1) (end 160.7 110.1) (width 0.762) (layer "B.Cu") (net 13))
 (segment (start 160.9 119.4) (end 159.9 119.4) (width 0.762) (layer "B.Cu") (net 13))
 (segment (start 161.1 94.3) (end 161.1 93.4) (width 0.762) (layer "B.Cu") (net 13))
 (segment (start 161.8 104.4) (end 162 104.6) (width 0.762) (layer "B.Cu") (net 13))
 (segment (start 162 109.1) (end 161 110.1) (width 0.762) (layer "B.Cu") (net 13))
 (segment (start 167.42406 119.4) (end 163.1 119.4) (width 0.762) (layer "B.Cu") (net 13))
 (segment (start 160.8 116.8) (end 161.9 116.8) (width 0.762) (layer "B.Cu") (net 13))
 (segment (start 162 119.4) (end 160.9 119.4) (width 0.762) (layer "B.Cu") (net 13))
 (segment (start 160.7 110.1) (end 162 110.1) (width 0.762) (layer "B.Cu") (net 13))
 (segment (start 161.9 94.2) (end 162 94.1) (width 0.762) (layer "B.Cu") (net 13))
 (segment (start 162 111.1) (end 162 110.1) (width 0.762) (layer "B.Cu") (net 13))
 (segment (start 161.1 93.4) (end 161.2 93.3) (width 0.762) (layer "B.Cu") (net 13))
 (segment (start 160.1 92.2) (end 158.825 92.2) (width 0.762) (layer "B.Cu") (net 13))
 (segment (start 162 116) (end 162 111.1) (width 0.762) (layer "B.Cu") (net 13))
 (segment (start 162 120.5) (end 163.1 119.4) (width 0.762) (layer "B.Cu") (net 13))
 (segment (start 162 95.2) (end 162 94.1) (width 0.762) (layer "B.Cu") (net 13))
 (segment (start 158.825 94.2) (end 161.1 94.2) (width 0.762) (layer "B.Cu") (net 13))
 (segment (start 163 126.6) (end 162 125.6) (width 0.762) (layer "B.Cu") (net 13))
 (segment (start 162 119.4) (end 162 118.3) (width 0.762) (layer "B.Cu") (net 13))
 (segment (start 158.825 116.8) (end 160.8 116.8) (width 0.762) (layer "B.Cu") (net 13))
 (segment (start 161.2 116.8) (end 162 116) (width 0.762) (layer "B.Cu") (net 13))
 (segment (start 162 94.1) (end 161.2 93.3) (width 0.762) (layer "B.Cu") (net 13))
 (segment (start 162 104.6) (end 162 99.8) (width 0.762) (layer "B.Cu") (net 13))
 (segment (start 162 120.5) (end 162 119.4) (width 0.762) (layer "B.Cu") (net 13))
 (segment (start 158.825 104.4) (end 161.8 104.4) (width 0.762) (layer "B.Cu") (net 13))
 (segment (start 162 117.6) (end 161.2 116.8) (width 0.762) (layer "B.Cu") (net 13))
 (segment (start 160.9 119.4) (end 162 118.3) (width 0.762) (layer "B.Cu") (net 13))
 (segment (start 163.1 119.4) (end 162 119.4) (width 0.762) (layer "B.Cu") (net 13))
 (segment (start 158.825 99.8) (end 162 99.8) (width 0.762) (layer "B.Cu") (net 13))
 (segment (start 134.6 103.4) (end 141.3 110.1) (width 0.762) (layer "B.Cu") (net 13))
 (segment (start 162 111.1) (end 161 110.1) (width 0.762) (layer "B.Cu") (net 13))
 (segment (start 169.07271 117.75135) (end 167.42406 119.4) (width 0.762) (layer "B.Cu") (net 13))
 (segment (start 160.9 119.4) (end 162 120.5) (width 0.762) (layer "B.Cu") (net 13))
 (segment (start 161.9 123.8) (end 162 123.8) (width 0.762) (layer "B.Cu") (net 13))
 (segment (start 162 123.8) (end 162 122.9) (width 0.762) (layer "B.Cu") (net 13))
 (segment (start 162 116.9) (end 162 116) (width 0.762) (layer "B.Cu") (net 13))
 (segment (start 118.875 125.2) (end 118.25 125.825) (width 0.762) (layer "F.Cu") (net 11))
 (segment (start 119.4 125.2) (end 118.875 125.2) (width 0.762) (layer "F.Cu") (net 11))
 (segment (start 118.875 125.2) (end 118.25 124.575) (width 0.762) (layer "F.Cu") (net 11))
 (via (at 119.4 125.2) (size 0.8) (drill 0.4) (layers "F.Cu" "B.Cu") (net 11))
 (segment (start 122.175 125.2) (end 119.4 125.2) (width 0.762) (layer "B.Cu") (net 11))
 (segment (start 136.075 119.4) (end 135.45 120.025) (width 0.762) (layer "F.Cu") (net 5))
 (segment (start 136.6 119.4) (end 136.075 119.4) (width 0.762) (layer "F.Cu") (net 5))
 (segment (start 136.075 119.4) (end 135.45 118.775) (width 0.762) (layer "F.Cu") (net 5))
 (via (at 136.6 119.4) (size 0.8) (drill 0.4) (layers "F.Cu" "B.Cu") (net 5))
 (segment (start 157.175 119.4) (end 136.6 119.4) (width 0.762) (layer "B.Cu") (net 5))
 (segment (start 155.8 116.8) (end 155.275 116.8) (width 0.762) (layer "F.Cu") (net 4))
 (segment (start 155.275 116.8) (end 154.65 116.175) (width 0.762) (layer "F.Cu") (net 4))
 (segment (start 155.275 116.8) (end 154.65 117.425) (width 0.762) (layer "F.Cu") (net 4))
 (via (at 155.8 116.8) (size 0.8) (drill 0.4) (layers "F.Cu" "B.Cu") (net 4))
 (segment (start 157.175 116.8) (end 155.8 116.8) (width 0.762) (layer "B.Cu") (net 4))
 (segment (start 167.9 126.6) (end 168.325 126.6) (width 0.762) (layer "F.Cu") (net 8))
 (segment (start 168.325 126.6) (end 168.95 127.225) (width 0.762) (layer "F.Cu") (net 8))
 (segment (start 168.325 126.6) (end 168.95 125.975) (width 0.762) (layer "F.Cu") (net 8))
 (via (at 167.9 126.6) (size 0.8) (drill 0.4) (layers "F.Cu" "B.Cu") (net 8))
 (segment (start 166.625 126.6) (end 167.9 126.6) (width 0.762) (layer "B.Cu") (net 8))
 (segment (start 155.725 97) (end 156.35 96.375) (width 0.762) (layer "F.Cu") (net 3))
 (segment (start 155.3 97) (end 155.725 97) (width 0.762) (layer "F.Cu") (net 3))
 (segment (start 155.725 97) (end 156.35 97.625) (width 0.762) (layer "F.Cu") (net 3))
 (via (at 155.3 97) (size 0.8) (drill 0.4) (layers "F.Cu" "B.Cu") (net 3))
 (segment (start 153.5 99) (end 153.5 98) (width 0.762) (layer "B.Cu") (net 3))
 (segment (start 157.175 99.8) (end 154.3 99.8) (width 0.762) (layer "B.Cu") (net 3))
 (segment (start 153.5 98) (end 154.5 97) (width 0.762) (layer "B.Cu") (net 3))
 (segment (start 154.5 97) (end 155.3 97) (width 0.762) (layer "B.Cu") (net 3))
 (segment (start 154.3 99.8) (end 153.5 99) (width 0.762) (layer "B.Cu") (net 3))
 (segment (start 169.8 127.2) (end 169.8 121.24346) (width 0.762) (layer "B.Cu") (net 14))
 (segment (start 169.8 121.24346) (end 170.960672 120.082788) (width 0.762) (layer "B.Cu") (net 14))
 (segment (start 167.75 129.25) (end 169.8 127.2) (width 0.762) (layer "B.Cu") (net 14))
 (segment (start 149.1 129.25) (end 167.75 129.25) (width 0.762) (layer "B.Cu") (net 14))
 (segment (start 146.2 49.3) (end 144.9 48) (width 0.762) (layer "B.Cu") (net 15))
 (segment (start 138.1 65.4) (end 138.1 70.75) (width 0.762) (layer "B.Cu") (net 15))
 (segment (start 146.2 63.4) (end 146.2 49.3) (width 0.762) (layer "B.Cu") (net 15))
 (segment (start 149.1 66.3) (end 146.2 63.4) (width 0.762) (layer "B.Cu") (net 15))
 (segment (start 149.1 70.75) (end 149.1 66.3) (width 0.762) (layer "B.Cu") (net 15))
 (segment (start 140.8 62.7) (end 138.1 65.4) (width 0.762) (layer "B.Cu") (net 15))
 (segment (start 140.8 49.4) (end 140.8 62.7) (width 0.762) (layer "B.Cu") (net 15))
 (segment (start 142.2 48) (end 140.8 49.4) (width 0.762) (layer "B.Cu") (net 15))
 (segment (start 144.9 48) (end 142.2 48) (width 0.762) (layer "B.Cu") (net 15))
 (segment (start 127.325 98.8) (end 127.95 98.175) (width 0.762) (layer "F.Cu") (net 6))
 (segment (start 126.9 98.8) (end 127.325 98.8) (width 0.762) (layer "F.Cu") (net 6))
 (segment (start 127.325 98.8) (end 127.95 99.425) (width 0.762) (layer "F.Cu") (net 6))
 (via (at 126.9 98.8) (size 0.8) (drill 0.4) (layers "F.Cu" "B.Cu") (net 6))
 (segment (start 125.1 102) (end 125.1 99.7) (width 0.762) (layer "B.Cu") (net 6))
 (segment (start 126 98.8) (end 126.9 98.8) (width 0.762) (layer "B.Cu") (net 6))
 (segment (start 125.1 99.7) (end 126 98.8) (width 0.762) (layer "B.Cu") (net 6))
 (segment (start 128.175 103.4) (end 126.5 103.4) (width 0.762) (layer "B.Cu") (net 6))
 (segment (start 126.5 103.4) (end 125.1 102) (width 0.762) (layer "B.Cu") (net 6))
 (segment (start 144.5 104.4) (end 144 104.4) (width 0.762) (layer "F.Cu") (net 9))
 (segment (start 144 104.4) (end 143.4 103.8) (width 0.762) (layer "F.Cu") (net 9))
 (segment (start 144.05 104.4) (end 143.4 105.05) (width 0.762) (layer "F.Cu") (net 9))
 (segment (start 144.5 104.4) (end 144.05 104.4) (width 0.762) (layer "F.Cu") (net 9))
 (via (at 144.5 104.4) (size 0.8) (drill 0.4) (layers "F.Cu" "B.Cu") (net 9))
 (segment (start 157.175 104.4) (end 144.5 104.4) (width 0.762) (layer "B.Cu") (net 9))
 (segment (start 146.4 87.6) (end 145.875 87.6) (width 0.762) (layer "F.Cu") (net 10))
 (segment (start 145.875 87.6) (end 145.25 86.975) (width 0.762) (layer "F.Cu") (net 10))
 (segment (start 145.875 87.6) (end 145.25 88.225) (width 0.762) (layer "F.Cu") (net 10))
 (via (at 146.4 87.6) (size 0.8) (drill 0.4) (layers "F.Cu" "B.Cu") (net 10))
 (segment (start 153 94.2) (end 149.3 90.5) (width 0.762) (layer "B.Cu") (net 10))
 (segment (start 157.175 94.2) (end 153 94.2) (width 0.762) (layer "B.Cu") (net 10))
 (segment (start 149.3 90.5) (end 146.4 87.6) (width 0.762) (layer "B.Cu") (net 10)))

